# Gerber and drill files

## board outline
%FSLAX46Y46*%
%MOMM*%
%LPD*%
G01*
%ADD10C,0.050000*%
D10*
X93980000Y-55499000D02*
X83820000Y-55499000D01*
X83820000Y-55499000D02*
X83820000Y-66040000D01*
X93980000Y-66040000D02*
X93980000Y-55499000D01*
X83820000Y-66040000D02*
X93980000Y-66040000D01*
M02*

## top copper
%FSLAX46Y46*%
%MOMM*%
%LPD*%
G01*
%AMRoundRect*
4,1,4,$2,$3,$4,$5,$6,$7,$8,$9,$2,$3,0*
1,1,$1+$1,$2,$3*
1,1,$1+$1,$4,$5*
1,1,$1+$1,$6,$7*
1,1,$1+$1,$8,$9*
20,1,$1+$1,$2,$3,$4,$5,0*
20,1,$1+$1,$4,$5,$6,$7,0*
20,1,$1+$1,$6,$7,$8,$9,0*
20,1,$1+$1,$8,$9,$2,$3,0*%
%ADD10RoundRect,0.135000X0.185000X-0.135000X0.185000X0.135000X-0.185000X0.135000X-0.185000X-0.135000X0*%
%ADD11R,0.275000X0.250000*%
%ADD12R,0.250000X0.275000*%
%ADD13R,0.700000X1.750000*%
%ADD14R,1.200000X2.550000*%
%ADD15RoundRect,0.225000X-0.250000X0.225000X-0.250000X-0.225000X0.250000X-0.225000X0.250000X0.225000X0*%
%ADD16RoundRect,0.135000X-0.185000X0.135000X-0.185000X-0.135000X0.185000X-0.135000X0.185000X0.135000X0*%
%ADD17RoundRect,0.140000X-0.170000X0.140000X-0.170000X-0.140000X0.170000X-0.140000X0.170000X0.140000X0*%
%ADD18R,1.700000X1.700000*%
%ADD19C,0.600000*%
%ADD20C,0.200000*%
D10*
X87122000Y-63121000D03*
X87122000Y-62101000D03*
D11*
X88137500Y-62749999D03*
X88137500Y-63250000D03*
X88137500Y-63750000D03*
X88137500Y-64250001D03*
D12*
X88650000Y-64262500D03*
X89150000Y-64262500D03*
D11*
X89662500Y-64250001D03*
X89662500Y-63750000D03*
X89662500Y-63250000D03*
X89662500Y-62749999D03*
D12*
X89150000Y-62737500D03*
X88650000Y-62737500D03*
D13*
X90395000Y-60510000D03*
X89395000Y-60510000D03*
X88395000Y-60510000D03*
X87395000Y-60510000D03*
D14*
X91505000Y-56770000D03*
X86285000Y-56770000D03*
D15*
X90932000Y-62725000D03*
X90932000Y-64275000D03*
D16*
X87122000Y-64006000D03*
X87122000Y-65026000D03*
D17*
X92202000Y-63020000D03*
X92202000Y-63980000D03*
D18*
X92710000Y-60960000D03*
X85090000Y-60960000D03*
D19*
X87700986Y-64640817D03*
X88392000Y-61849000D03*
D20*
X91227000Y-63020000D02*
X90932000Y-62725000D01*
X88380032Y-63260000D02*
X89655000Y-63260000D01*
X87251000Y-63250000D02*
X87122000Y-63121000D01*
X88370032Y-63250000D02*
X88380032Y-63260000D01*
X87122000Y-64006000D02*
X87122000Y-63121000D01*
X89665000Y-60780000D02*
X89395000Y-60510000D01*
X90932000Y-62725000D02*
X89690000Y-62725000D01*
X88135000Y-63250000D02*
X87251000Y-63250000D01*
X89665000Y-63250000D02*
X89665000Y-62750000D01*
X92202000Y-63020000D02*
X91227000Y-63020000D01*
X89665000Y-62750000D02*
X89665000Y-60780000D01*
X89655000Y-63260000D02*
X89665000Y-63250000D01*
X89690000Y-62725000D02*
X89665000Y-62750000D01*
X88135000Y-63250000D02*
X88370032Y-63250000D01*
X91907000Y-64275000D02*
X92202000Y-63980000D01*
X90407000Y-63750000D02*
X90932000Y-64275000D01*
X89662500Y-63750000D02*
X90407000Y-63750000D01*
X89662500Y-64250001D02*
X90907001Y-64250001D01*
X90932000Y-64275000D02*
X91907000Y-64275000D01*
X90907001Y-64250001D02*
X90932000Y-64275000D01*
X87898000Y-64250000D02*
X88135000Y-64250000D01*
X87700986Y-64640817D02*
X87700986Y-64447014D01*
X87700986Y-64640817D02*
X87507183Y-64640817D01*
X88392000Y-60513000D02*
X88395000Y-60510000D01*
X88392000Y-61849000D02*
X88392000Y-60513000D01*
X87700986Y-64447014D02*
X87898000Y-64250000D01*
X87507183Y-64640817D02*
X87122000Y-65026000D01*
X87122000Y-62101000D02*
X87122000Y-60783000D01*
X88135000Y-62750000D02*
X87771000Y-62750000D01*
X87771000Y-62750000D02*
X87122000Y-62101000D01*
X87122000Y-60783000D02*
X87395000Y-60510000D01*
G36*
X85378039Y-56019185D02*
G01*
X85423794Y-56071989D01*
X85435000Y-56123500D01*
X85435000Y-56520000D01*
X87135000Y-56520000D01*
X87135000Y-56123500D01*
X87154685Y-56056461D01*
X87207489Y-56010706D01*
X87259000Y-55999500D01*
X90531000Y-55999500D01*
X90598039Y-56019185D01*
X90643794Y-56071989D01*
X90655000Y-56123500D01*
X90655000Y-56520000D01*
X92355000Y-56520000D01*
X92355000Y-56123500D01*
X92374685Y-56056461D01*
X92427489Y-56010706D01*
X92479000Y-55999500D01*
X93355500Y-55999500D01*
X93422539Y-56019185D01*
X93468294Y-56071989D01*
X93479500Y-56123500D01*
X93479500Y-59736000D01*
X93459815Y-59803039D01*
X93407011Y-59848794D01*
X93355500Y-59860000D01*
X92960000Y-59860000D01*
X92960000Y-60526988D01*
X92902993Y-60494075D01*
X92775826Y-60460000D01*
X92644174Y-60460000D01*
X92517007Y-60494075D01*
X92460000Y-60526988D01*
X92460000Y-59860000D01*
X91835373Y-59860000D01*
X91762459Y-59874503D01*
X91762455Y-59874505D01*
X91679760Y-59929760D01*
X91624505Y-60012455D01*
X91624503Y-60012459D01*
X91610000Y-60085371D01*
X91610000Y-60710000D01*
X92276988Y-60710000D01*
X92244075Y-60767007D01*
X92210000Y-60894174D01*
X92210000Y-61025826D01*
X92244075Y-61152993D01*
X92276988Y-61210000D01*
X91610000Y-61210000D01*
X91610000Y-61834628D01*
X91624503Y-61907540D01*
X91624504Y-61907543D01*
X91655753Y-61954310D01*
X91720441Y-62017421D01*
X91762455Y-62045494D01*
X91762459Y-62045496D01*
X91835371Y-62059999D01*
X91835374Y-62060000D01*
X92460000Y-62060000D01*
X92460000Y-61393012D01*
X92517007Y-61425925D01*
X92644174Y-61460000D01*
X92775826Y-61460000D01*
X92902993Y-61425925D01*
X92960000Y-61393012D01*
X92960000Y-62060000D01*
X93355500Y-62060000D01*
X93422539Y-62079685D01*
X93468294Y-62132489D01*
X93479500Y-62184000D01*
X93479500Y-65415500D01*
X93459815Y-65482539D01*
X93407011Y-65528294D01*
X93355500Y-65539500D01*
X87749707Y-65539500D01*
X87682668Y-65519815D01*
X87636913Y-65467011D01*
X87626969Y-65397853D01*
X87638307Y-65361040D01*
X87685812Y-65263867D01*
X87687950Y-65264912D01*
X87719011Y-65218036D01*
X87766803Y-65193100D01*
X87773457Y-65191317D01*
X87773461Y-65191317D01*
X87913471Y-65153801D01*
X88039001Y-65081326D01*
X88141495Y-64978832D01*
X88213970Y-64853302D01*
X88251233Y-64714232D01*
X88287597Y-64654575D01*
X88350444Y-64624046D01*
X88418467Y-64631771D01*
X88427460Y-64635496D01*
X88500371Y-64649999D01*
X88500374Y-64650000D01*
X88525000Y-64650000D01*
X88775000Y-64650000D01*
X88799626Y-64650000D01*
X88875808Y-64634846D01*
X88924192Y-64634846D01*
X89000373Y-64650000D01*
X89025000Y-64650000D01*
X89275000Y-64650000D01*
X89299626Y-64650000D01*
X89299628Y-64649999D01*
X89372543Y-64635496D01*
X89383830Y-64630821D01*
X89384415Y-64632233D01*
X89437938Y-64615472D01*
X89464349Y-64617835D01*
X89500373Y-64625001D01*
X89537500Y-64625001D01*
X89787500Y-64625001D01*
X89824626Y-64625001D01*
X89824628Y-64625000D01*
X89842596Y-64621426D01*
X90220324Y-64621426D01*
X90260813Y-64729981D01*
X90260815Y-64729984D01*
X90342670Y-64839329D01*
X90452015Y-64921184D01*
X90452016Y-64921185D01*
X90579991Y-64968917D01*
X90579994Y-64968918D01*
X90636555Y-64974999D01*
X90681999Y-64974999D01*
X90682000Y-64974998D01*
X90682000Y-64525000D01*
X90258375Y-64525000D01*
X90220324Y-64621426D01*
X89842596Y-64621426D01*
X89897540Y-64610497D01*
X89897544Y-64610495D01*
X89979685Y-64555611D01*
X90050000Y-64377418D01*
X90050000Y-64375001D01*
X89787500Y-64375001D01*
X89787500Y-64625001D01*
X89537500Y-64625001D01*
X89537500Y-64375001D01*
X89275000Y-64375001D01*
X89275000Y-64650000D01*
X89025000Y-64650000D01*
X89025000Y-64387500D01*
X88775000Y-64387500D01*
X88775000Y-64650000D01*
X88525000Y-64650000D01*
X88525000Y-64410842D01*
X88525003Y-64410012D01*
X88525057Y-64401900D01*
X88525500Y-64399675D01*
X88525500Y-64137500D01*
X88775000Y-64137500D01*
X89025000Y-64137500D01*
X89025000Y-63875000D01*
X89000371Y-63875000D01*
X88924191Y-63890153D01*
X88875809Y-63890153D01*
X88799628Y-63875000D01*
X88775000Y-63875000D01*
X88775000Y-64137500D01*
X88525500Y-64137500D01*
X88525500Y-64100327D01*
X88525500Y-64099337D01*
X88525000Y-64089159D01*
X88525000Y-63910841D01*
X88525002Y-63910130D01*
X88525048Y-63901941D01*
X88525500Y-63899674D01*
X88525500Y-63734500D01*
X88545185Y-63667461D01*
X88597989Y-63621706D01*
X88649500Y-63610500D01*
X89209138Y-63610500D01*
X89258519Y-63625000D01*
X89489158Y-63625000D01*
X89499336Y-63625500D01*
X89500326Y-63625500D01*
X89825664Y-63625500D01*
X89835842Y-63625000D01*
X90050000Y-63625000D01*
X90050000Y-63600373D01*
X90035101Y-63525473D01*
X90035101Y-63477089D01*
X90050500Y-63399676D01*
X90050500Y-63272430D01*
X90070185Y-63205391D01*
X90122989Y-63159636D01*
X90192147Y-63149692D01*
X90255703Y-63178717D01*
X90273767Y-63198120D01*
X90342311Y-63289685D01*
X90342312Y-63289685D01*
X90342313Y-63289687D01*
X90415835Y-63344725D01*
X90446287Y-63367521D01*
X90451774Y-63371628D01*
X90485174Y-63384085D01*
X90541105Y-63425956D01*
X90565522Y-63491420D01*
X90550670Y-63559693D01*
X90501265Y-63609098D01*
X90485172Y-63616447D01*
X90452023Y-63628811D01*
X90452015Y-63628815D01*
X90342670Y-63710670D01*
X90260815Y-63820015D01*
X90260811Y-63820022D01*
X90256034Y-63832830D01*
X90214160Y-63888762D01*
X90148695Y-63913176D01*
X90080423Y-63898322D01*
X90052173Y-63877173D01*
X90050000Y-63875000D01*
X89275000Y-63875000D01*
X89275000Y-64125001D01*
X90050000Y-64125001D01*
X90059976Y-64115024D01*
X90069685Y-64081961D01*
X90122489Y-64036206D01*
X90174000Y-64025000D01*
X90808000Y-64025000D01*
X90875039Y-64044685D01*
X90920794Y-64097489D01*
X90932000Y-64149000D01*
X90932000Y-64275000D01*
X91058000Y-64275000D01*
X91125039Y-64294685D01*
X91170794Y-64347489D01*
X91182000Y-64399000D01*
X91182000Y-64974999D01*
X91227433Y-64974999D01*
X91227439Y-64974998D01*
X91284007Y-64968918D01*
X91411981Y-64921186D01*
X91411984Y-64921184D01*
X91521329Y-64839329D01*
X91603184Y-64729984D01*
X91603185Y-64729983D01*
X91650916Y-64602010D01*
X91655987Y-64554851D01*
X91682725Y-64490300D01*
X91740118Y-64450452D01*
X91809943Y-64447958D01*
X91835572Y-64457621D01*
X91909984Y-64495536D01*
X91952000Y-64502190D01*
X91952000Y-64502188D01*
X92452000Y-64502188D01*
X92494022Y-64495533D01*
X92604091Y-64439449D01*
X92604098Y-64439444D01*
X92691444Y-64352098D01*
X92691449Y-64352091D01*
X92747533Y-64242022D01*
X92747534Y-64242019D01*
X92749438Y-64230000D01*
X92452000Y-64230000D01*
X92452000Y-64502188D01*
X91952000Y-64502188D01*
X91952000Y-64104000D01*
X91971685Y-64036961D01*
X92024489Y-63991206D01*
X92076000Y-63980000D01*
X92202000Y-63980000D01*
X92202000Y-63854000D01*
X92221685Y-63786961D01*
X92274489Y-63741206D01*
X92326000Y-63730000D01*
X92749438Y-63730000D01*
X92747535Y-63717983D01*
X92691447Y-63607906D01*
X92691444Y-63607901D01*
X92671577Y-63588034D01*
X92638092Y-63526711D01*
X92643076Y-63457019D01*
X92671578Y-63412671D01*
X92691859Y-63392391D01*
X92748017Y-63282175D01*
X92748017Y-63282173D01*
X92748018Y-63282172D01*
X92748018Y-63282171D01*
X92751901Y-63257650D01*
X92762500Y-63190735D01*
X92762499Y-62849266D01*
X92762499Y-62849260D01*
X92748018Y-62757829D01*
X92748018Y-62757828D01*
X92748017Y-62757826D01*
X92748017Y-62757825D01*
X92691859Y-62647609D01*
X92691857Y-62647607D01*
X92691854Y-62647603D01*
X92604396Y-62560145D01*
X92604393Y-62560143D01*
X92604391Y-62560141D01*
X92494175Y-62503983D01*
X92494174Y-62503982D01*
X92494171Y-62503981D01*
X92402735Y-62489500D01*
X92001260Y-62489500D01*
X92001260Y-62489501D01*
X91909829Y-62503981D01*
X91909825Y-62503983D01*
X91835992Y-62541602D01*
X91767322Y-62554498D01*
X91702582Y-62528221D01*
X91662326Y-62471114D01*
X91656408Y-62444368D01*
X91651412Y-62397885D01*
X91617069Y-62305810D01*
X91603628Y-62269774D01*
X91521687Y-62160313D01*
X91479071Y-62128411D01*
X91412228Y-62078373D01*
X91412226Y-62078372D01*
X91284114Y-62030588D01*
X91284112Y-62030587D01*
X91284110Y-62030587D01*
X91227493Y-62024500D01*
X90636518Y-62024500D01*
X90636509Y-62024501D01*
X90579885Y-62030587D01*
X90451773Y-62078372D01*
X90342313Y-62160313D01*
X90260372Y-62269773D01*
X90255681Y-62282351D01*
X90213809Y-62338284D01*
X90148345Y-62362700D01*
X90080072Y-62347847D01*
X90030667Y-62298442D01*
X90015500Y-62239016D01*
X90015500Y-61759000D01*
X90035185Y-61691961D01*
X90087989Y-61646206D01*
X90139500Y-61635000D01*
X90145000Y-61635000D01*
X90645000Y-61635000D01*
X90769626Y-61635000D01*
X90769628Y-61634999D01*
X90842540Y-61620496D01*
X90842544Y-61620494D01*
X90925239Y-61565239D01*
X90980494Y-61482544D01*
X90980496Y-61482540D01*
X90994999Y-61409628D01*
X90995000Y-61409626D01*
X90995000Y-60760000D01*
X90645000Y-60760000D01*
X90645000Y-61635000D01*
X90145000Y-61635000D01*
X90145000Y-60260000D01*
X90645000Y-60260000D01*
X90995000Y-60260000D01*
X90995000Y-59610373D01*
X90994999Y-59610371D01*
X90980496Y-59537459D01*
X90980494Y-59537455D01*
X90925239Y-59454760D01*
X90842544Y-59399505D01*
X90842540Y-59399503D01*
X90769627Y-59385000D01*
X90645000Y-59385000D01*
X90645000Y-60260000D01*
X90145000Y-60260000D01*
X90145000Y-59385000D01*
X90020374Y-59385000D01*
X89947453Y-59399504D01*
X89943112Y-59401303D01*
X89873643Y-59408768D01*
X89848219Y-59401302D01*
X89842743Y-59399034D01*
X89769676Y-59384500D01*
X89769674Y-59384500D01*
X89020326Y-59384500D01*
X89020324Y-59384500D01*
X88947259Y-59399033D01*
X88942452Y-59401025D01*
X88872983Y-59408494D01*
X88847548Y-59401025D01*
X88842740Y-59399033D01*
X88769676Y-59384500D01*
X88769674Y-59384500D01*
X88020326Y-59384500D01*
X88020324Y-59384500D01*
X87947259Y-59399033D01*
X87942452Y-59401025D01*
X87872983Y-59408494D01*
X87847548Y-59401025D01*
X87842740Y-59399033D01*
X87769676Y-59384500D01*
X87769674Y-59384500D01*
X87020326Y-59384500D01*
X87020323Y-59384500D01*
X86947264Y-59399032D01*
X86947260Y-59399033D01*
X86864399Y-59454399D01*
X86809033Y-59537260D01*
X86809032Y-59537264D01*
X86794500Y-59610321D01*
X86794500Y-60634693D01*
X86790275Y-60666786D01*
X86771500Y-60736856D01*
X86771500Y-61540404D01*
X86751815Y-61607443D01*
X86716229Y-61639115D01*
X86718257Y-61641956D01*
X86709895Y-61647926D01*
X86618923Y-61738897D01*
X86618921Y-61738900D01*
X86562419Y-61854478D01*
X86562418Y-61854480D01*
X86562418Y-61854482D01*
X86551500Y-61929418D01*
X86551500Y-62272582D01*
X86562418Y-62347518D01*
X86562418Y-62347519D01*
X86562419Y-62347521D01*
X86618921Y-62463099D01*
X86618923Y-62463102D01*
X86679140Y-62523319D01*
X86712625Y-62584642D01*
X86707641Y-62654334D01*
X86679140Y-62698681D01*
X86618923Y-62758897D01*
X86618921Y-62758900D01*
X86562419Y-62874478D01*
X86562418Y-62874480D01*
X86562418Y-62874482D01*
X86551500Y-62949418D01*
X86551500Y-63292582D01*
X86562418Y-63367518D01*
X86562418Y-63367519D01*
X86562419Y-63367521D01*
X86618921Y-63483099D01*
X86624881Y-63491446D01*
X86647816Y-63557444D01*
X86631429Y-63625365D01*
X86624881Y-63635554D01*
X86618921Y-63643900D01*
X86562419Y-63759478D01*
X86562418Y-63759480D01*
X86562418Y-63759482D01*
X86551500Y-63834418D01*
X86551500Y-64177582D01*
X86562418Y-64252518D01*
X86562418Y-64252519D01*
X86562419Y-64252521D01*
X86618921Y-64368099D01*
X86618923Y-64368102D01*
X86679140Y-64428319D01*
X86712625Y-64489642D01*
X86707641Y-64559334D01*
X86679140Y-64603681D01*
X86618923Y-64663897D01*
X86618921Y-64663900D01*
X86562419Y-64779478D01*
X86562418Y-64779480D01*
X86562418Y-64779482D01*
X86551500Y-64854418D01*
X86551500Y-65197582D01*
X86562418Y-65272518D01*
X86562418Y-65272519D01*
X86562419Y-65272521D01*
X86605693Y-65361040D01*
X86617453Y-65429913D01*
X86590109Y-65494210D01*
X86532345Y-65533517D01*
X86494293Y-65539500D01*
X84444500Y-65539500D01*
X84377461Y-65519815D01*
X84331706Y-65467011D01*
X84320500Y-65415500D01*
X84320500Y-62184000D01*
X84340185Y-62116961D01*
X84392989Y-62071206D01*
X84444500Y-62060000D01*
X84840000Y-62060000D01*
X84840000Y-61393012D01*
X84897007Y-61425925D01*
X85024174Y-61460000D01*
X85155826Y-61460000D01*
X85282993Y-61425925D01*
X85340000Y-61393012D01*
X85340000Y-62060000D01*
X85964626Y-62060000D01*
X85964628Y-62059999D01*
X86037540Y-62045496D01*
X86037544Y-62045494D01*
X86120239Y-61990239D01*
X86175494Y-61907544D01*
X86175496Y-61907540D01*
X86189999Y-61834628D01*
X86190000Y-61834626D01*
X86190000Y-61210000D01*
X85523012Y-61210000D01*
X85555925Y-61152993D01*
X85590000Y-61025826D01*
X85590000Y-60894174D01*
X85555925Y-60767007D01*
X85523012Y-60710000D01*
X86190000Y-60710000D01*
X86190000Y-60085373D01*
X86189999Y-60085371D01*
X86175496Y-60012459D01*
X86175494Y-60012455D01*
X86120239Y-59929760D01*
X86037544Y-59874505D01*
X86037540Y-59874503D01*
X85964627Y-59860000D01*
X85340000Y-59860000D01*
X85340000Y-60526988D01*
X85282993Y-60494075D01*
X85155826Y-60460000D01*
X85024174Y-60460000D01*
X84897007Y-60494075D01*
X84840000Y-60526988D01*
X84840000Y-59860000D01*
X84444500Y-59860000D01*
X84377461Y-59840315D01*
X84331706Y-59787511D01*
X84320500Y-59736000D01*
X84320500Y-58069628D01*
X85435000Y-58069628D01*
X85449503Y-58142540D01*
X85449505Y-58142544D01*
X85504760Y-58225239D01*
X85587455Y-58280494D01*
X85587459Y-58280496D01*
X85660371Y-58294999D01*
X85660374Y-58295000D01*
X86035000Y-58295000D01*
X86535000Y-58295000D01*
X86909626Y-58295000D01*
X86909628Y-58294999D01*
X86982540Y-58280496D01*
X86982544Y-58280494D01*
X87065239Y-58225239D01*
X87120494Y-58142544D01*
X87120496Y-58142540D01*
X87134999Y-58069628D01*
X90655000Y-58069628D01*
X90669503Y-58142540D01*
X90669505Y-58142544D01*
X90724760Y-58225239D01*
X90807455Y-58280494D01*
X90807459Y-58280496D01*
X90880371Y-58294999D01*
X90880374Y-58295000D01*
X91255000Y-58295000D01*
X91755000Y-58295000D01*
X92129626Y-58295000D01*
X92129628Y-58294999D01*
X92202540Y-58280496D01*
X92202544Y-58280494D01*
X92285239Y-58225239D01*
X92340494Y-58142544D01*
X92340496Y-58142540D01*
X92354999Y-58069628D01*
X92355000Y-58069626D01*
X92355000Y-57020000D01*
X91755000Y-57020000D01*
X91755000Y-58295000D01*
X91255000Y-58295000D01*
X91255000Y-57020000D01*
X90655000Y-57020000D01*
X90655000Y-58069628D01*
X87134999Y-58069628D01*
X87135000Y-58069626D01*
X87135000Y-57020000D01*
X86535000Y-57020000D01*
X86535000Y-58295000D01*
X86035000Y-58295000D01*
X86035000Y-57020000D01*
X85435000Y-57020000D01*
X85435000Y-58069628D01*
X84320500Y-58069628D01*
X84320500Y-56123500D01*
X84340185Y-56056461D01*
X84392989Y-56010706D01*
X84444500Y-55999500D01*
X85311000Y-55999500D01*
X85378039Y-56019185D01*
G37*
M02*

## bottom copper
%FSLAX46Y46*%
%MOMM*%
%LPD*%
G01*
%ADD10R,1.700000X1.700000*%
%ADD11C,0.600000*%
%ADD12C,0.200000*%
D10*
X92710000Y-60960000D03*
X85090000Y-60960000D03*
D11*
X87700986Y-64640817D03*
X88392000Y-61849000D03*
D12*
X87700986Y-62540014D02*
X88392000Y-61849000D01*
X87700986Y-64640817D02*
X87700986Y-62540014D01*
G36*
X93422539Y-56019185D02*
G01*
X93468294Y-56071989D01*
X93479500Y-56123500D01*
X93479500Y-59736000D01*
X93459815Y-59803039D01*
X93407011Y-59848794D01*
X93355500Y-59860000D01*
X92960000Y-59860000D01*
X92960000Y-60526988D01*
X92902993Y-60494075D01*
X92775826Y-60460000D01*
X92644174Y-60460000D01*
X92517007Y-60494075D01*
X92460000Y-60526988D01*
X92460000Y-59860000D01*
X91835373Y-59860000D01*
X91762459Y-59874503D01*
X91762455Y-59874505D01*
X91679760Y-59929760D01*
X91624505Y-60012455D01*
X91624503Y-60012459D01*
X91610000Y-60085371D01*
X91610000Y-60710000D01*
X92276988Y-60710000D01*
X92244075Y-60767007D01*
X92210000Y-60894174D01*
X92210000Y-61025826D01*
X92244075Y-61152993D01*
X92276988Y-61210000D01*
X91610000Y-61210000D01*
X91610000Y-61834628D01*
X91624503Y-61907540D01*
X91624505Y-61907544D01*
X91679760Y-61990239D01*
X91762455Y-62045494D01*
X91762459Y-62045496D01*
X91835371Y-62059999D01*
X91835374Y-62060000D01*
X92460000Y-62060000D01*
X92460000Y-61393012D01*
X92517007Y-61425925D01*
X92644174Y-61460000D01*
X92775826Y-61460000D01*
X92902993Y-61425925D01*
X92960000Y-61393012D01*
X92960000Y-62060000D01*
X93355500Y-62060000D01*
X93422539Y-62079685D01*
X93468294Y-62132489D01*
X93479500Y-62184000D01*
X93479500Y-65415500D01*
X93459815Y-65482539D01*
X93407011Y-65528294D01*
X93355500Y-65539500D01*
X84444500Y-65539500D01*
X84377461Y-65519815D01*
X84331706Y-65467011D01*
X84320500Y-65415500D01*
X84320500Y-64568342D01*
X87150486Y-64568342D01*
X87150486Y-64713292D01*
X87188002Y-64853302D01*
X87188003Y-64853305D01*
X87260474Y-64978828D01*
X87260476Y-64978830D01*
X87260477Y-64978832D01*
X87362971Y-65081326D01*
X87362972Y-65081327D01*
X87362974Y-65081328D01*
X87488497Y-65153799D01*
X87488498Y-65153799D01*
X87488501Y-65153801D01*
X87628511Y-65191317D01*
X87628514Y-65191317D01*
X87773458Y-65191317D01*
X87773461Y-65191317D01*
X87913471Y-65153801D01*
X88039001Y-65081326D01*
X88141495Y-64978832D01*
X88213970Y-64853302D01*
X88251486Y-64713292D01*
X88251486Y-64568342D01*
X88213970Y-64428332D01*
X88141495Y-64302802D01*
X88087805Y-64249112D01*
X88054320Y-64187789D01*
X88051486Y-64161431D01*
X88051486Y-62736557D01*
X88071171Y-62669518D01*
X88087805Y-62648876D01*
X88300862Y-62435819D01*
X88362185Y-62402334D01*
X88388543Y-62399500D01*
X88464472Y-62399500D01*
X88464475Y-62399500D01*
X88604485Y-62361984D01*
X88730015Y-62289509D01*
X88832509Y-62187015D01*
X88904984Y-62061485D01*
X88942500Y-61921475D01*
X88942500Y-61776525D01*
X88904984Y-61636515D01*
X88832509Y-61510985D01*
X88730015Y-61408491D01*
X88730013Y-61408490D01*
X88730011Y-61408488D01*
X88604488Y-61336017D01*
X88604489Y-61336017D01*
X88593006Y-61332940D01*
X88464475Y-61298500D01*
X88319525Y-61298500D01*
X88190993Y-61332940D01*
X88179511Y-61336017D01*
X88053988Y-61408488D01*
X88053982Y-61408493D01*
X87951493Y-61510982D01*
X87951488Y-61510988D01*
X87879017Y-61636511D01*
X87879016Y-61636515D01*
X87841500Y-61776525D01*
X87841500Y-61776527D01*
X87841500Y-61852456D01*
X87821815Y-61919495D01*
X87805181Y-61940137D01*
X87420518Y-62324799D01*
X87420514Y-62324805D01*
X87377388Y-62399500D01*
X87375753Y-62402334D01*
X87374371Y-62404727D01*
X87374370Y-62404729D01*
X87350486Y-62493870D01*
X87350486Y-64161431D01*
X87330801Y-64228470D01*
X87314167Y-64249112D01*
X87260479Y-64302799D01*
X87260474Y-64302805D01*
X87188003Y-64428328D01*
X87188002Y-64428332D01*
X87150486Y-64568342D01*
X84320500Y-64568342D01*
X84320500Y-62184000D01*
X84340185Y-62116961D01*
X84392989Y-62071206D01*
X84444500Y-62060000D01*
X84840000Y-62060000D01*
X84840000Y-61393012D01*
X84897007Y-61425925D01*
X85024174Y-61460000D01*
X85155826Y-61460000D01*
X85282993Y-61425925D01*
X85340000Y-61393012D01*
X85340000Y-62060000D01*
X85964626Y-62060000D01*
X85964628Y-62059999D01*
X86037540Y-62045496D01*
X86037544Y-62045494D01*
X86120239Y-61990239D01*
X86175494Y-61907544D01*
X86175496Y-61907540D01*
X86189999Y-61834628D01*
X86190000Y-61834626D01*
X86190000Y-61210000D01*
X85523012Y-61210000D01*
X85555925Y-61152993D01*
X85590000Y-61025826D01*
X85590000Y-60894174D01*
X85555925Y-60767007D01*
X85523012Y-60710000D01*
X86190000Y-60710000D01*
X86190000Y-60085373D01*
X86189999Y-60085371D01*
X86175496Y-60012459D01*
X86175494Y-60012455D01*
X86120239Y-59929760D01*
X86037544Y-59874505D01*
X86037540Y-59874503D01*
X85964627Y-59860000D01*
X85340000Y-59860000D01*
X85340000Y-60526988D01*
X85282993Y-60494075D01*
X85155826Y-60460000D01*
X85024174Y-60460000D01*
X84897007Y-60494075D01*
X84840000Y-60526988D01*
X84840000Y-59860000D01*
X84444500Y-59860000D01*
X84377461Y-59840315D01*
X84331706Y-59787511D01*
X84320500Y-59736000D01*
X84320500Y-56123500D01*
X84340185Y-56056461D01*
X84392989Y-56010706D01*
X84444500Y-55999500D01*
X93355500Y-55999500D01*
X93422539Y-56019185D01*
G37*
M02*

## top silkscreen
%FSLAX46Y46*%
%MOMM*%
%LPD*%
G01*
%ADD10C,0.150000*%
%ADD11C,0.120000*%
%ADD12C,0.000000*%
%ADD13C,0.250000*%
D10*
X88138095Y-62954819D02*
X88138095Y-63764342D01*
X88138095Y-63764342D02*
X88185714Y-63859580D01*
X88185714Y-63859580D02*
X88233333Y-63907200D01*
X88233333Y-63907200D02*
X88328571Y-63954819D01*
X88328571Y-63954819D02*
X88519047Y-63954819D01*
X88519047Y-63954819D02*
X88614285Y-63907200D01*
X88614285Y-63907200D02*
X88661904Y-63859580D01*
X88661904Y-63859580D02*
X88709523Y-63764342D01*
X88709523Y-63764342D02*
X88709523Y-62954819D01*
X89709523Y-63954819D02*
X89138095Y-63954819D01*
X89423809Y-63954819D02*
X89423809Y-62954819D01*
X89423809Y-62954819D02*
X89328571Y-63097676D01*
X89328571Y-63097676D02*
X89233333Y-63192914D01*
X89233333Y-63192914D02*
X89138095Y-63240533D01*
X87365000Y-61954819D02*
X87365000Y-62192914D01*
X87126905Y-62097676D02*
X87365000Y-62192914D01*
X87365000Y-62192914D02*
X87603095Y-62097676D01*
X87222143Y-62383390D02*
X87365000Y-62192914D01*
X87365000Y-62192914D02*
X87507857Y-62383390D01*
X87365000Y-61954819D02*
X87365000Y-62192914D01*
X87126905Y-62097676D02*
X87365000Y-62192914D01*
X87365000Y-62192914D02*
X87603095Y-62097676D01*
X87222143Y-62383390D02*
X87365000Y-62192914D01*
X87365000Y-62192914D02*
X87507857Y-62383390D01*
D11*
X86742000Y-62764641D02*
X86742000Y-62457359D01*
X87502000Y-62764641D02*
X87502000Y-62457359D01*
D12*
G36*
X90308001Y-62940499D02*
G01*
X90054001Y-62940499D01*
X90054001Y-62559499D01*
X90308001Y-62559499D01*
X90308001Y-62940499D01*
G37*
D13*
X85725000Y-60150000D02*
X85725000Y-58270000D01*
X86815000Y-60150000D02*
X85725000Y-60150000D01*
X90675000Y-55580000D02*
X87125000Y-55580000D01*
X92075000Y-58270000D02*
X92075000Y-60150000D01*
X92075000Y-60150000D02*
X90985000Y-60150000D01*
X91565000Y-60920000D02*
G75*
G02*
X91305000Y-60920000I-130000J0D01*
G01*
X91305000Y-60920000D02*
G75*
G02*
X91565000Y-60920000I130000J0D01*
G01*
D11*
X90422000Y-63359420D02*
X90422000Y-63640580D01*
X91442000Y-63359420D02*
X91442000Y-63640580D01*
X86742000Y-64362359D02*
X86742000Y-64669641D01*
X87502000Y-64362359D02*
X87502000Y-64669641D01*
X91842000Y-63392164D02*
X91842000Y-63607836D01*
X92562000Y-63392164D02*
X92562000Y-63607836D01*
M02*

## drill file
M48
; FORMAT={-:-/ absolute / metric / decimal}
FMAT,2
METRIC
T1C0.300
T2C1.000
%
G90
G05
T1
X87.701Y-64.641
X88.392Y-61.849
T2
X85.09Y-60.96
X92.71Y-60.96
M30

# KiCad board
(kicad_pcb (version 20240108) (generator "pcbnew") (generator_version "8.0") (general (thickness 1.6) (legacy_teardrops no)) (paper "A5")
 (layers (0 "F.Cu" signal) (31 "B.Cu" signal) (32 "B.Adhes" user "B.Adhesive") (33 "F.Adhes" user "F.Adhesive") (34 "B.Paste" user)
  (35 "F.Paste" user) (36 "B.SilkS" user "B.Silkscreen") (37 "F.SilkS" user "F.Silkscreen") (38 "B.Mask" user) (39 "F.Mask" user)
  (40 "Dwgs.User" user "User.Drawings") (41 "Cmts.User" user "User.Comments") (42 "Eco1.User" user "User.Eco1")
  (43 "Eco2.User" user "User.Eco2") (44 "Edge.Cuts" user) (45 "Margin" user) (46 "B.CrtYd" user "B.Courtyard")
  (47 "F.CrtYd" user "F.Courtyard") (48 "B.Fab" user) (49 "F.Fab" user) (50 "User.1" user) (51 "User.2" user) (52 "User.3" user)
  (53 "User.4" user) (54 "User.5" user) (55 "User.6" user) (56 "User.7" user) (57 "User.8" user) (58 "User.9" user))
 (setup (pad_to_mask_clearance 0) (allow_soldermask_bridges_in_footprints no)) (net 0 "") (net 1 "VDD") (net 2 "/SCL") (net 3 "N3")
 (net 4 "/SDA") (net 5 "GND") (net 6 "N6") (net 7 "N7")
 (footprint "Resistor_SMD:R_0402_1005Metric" (layer "F.Cu") (at 87.122 62.611 90)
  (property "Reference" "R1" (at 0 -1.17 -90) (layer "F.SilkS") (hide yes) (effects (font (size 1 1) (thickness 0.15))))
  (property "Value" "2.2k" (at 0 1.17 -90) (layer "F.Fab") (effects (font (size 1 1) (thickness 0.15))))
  (fp_line (start -0.153641 -0.38) (end 0.153641 -0.38) (stroke (width 0.12) (type solid)) (layer "F.SilkS"))
  (fp_line (start -0.153641 0.38) (end 0.153641 0.38) (stroke (width 0.12) (type solid)) (layer "F.SilkS"))
  (pad "1" smd roundrect (at -0.51 0 90) (size 0.54 0.64) (layers "F.Cu" "F.Paste" "F.Mask") (roundrect_rratio 0.25) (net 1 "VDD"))
  (pad "2" smd roundrect (at 0.51 0 90) (size 0.54 0.64) (layers "F.Cu" "F.Paste" "F.Mask") (roundrect_rratio 0.25) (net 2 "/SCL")))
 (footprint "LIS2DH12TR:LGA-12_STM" (layer "F.Cu") (at 88.9 63.5)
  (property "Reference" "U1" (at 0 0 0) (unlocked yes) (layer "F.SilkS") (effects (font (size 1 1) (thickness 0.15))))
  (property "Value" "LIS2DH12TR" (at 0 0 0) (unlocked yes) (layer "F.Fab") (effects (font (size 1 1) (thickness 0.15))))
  (fp_poly
   (pts (xy 1.408001 -0.940501) (xy 1.408001 -0.559501) (xy 1.154001 -0.559501) (xy 1.154001 -0.940501)) (stroke (width 0) (type solid))
   (fill solid) (layer "F.SilkS"))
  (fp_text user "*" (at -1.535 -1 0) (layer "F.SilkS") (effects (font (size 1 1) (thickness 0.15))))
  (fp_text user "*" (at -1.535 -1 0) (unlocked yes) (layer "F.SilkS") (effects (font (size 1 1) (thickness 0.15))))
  (pad "1" smd rect (at -0.7625 -0.750001 90) (size 0.25 0.275) (layers "F.Cu" "F.Paste" "F.Mask") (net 2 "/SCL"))
  (pad "2" smd rect (at -0.7625 -0.25 90) (size 0.25 0.275) (layers "F.Cu" "F.Paste" "F.Mask") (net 1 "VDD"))
  (pad "3" smd rect (at -0.7625 0.25 90) (size 0.25 0.275) (layers "F.Cu" "F.Paste" "F.Mask") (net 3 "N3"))
  (pad "4" smd rect (at -0.7625 0.750001 90) (size 0.25 0.275) (layers "F.Cu" "F.Paste" "F.Mask") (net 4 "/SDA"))
  (pad "5" smd rect (at -0.25 0.7625) (size 0.25 0.275) (layers "F.Cu" "F.Paste" "F.Mask") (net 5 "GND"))
  (pad "6" smd rect (at 0.25 0.7625) (size 0.25 0.275) (layers "F.Cu" "F.Paste" "F.Mask") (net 5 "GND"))
  (pad "7" smd rect (at 0.7625 0.750001 90) (size 0.25 0.275) (layers "F.Cu" "F.Paste" "F.Mask") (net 5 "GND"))
  (pad "8" smd rect (at 0.7625 0.25 90) (size 0.25 0.275) (layers "F.Cu" "F.Paste" "F.Mask") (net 5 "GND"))
  (pad "9" smd rect (at 0.7625 -0.25 90) (size 0.25 0.275) (layers "F.Cu" "F.Paste" "F.Mask") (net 1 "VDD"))
  (pad "10" smd rect (at 0.7625 -0.750001 90) (size 0.25 0.275) (layers "F.Cu" "F.Paste" "F.Mask") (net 1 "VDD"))
  (pad "11" smd rect (at 0.25 -0.7625) (size 0.25 0.275) (layers "F.Cu" "F.Paste" "F.Mask") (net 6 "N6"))
  (pad "12" smd rect (at -0.25 -0.7625) (size 0.25 0.275) (layers "F.Cu" "F.Paste" "F.Mask") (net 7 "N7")))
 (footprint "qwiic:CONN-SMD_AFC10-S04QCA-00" (layer "F.Cu") (at 88.895 58.64 180)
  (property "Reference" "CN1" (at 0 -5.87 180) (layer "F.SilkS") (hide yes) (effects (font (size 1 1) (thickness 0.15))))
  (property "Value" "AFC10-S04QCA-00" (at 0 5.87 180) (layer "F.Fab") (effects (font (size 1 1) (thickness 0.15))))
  (fp_line (start 3.17 -1.51) (end 3.17 0.37) (stroke (width 0.25) (type solid)) (layer "F.SilkS"))
  (fp_line (start 2.08 -1.51) (end 3.17 -1.51) (stroke (width 0.25) (type solid)) (layer "F.SilkS"))
  (fp_line (start -1.78 3.06) (end 1.77 3.06) (stroke (width 0.25) (type solid)) (layer "F.SilkS"))
  (fp_line (start -3.18 0.37) (end -3.18 -1.51) (stroke (width 0.25) (type solid)) (layer "F.SilkS"))
  (fp_line (start -3.18 -1.51) (end -2.09 -1.51) (stroke (width 0.25) (type solid)) (layer "F.SilkS"))
  (fp_circle (center -2.54 -2.28) (end -2.41 -2.28) (stroke (width 0.25) (type solid)) (fill none) (layer "F.SilkS"))
  (pad "1" smd rect (at -1.5 -1.87 180) (size 0.7 1.75) (layers "F.Cu" "F.Paste" "F.Mask") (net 5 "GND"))
  (pad "2" smd rect (at -0.5 -1.87 180) (size 0.7 1.75) (layers "F.Cu" "F.Paste" "F.Mask") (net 1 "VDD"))
  (pad "3" smd rect (at 0.5 -1.87 180) (size 0.7 1.75) (layers "F.Cu" "F.Paste" "F.Mask") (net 4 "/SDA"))
  (pad "4" smd rect (at 1.5 -1.87 180) (size 0.7 1.75) (layers "F.Cu" "F.Paste" "F.Mask") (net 2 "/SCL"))
  (pad "5" smd rect (at -2.61 1.87 180) (size 1.2 2.55) (layers "F.Cu" "F.Paste" "F.Mask") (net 5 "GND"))
  (pad "6" smd rect (at 2.61 1.87 180) (size 1.2 2.55) (layers "F.Cu" "F.Paste" "F.Mask") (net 5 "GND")))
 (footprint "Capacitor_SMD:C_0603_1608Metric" (layer "F.Cu") (at 90.932 63.5 -90)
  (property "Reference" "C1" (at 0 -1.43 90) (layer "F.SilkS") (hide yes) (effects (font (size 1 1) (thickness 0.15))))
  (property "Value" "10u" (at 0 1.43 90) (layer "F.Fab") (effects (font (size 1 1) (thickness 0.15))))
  (fp_line (start -0.14058 0.51) (end 0.14058 0.51) (stroke (width 0.12) (type solid)) (layer "F.SilkS"))
  (fp_line (start -0.14058 -0.51) (end 0.14058 -0.51) (stroke (width 0.12) (type solid)) (layer "F.SilkS"))
  (pad "1" smd roundrect (at -0.775 0 270) (size 0.9 0.95) (layers "F.Cu" "F.Paste" "F.Mask") (roundrect_rratio 0.25) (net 1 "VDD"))
  (pad "2" smd roundrect (at 0.775 0 270) (size 0.9 0.95) (layers "F.Cu" "F.Paste" "F.Mask") (roundrect_rratio 0.25) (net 5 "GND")))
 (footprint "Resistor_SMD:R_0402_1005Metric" (layer "F.Cu") (at 87.122 64.516 -90)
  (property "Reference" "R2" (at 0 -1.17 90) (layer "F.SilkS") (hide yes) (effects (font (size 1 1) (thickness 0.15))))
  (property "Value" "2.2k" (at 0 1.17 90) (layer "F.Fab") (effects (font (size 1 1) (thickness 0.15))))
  (fp_line (start -0.153641 0.38) (end 0.153641 0.38) (stroke (width 0.12) (type solid)) (layer "F.SilkS"))
  (fp_line (start -0.153641 -0.38) (end 0.153641 -0.38) (stroke (width 0.12) (type solid)) (layer "F.SilkS"))
  (pad "1" smd roundrect (at -0.51 0 270) (size 0.54 0.64) (layers "F.Cu" "F.Paste" "F.Mask") (roundrect_rratio 0.25) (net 1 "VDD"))
  (pad "2" smd roundrect (at 0.51 0 270) (size 0.54 0.64) (layers "F.Cu" "F.Paste" "F.Mask") (roundrect_rratio 0.25) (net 4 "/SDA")))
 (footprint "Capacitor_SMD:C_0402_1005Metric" (layer "F.Cu") (at 92.202 63.5 -90)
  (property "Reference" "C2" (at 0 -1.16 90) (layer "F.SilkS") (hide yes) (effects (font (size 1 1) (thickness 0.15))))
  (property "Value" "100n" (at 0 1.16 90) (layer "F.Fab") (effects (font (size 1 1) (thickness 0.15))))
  (fp_line (start -0.107836 0.36) (end 0.107836 0.36) (stroke (width 0.12) (type solid)) (layer "F.SilkS"))
  (fp_line (start -0.107836 -0.36) (end 0.107836 -0.36) (stroke (width 0.12) (type solid)) (layer "F.SilkS"))
  (pad "1" smd roundrect (at -0.48 0 270) (size 0.56 0.62) (layers "F.Cu" "F.Paste" "F.Mask") (roundrect_rratio 0.25) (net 1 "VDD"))
  (pad "2" smd roundrect (at 0.48 0 270) (size 0.56 0.62) (layers "F.Cu" "F.Paste" "F.Mask") (roundrect_rratio 0.25) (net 5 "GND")))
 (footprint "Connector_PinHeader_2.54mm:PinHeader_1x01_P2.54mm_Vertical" (layer "B.Cu") (at 92.71 60.96 180)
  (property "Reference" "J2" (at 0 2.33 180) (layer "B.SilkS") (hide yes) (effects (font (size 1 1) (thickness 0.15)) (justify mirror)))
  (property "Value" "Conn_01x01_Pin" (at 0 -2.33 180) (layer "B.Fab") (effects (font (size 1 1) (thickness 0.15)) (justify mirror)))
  (pad "1" thru_hole rect (at 0 0 180) (size 1.7 1.7) (drill 1) (layers "*.Cu" "*.Mask") (remove_unused_layers no) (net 5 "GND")))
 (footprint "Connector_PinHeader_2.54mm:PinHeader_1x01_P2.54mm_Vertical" (layer "B.Cu") (at 85.09 60.96 180)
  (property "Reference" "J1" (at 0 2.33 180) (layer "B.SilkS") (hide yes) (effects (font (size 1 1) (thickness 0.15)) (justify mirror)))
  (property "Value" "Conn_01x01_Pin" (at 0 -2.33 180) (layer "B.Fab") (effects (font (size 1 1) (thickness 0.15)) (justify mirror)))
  (pad "1" thru_hole rect (at 0 0 180) (size 1.7 1.7) (drill 1) (layers "*.Cu" "*.Mask") (remove_unused_layers no) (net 5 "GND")))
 (gr_line (start 93.98 55.499) (end 83.82 55.499) (stroke (width 0.05) (type default)) (layer "Edge.Cuts"))
 (gr_line (start 83.82 55.499) (end 83.82 66.04) (stroke (width 0.05) (type default)) (layer "Edge.Cuts"))
 (gr_line (start 93.98 66.04) (end 93.98 55.499) (stroke (width 0.05) (type default)) (layer "Edge.Cuts"))
 (gr_line (start 83.82 66.04) (end 93.98 66.04) (stroke (width 0.05) (type default)) (layer "Edge.Cuts"))
 (segment (start 91.227 63.02) (end 90.932 62.725) (width 0.2) (layer "F.Cu") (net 1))
 (segment (start 88.380032 63.26) (end 89.655 63.26) (width 0.2) (layer "F.Cu") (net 1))
 (segment (start 87.251 63.25) (end 87.122 63.121) (width 0.2) (layer "F.Cu") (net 1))
 (segment (start 88.370032 63.25) (end 88.380032 63.26) (width 0.2) (layer "F.Cu") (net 1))
 (segment (start 87.122 64.006) (end 87.122 63.121) (width 0.2) (layer "F.Cu") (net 1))
 (segment (start 89.665 60.78) (end 89.395 60.51) (width 0.2) (layer "F.Cu") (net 1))
 (segment (start 90.932 62.725) (end 89.69 62.725) (width 0.2) (layer "F.Cu") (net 1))
 (segment (start 88.135 63.25) (end 87.251 63.25) (width 0.2) (layer "F.Cu") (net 1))
 (segment (start 89.665 63.25) (end 89.665 62.75) (width 0.2) (layer "F.Cu") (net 1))
 (segment (start 92.202 63.02) (end 91.227 63.02) (width 0.2) (layer "F.Cu") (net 1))
 (segment (start 89.665 62.75) (end 89.665 60.78) (width 0.2) (layer "F.Cu") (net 1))
 (segment (start 89.655 63.26) (end 89.665 63.25) (width 0.2) (layer "F.Cu") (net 1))
 (segment (start 89.69 62.725) (end 89.665 62.75) (width 0.2) (layer "F.Cu") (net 1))
 (segment (start 88.135 63.25) (end 88.370032 63.25) (width 0.2) (layer "F.Cu") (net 1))
 (segment (start 91.907 64.275) (end 92.202 63.98) (width 0.2) (layer "F.Cu") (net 5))
 (segment (start 90.407 63.75) (end 90.932 64.275) (width 0.2) (layer "F.Cu") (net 5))
 (segment (start 89.6625 63.75) (end 90.407 63.75) (width 0.2) (layer "F.Cu") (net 5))
 (segment (start 89.6625 64.250001) (end 90.907001 64.250001) (width 0.2) (layer "F.Cu") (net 5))
 (segment (start 90.932 64.275) (end 91.907 64.275) (width 0.2) (layer "F.Cu") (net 5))
 (segment (start 90.907001 64.250001) (end 90.932 64.275) (width 0.2) (layer "F.Cu") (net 5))
 (segment (start 87.898 64.25) (end 88.135 64.25) (width 0.2) (layer "F.Cu") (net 4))
 (segment (start 87.700986 64.640817) (end 87.700986 64.447014) (width 0.2) (layer "F.Cu") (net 4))
 (segment (start 87.700986 64.640817) (end 87.507183 64.640817) (width 0.2) (layer "F.Cu") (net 4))
 (segment (start 88.392 60.513) (end 88.395 60.51) (width 0.2) (layer "F.Cu") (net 4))
 (segment (start 88.392 61.849) (end 88.392 60.513) (width 0.2) (layer "F.Cu") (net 4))
 (segment (start 87.700986 64.447014) (end 87.898 64.25) (width 0.2) (layer "F.Cu") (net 4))
 (segment (start 87.507183 64.640817) (end 87.122 65.026) (width 0.2) (layer "F.Cu") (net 4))
 (via (at 87.700986 64.640817) (size 0.6) (drill 0.3) (layers "F.Cu" "B.Cu") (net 4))
 (via (at 88.392 61.849) (size 0.6) (drill 0.3) (layers "F.Cu" "B.Cu") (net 4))
 (segment (start 87.700986 62.540014) (end 88.392 61.849) (width 0.2) (layer "B.Cu") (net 4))
 (segment (start 87.700986 64.640817) (end 87.700986 62.540014) (width 0.2) (layer "B.Cu") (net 4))
 (segment (start 87.122 62.101) (end 87.122 60.783) (width 0.2) (layer "F.Cu") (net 2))
 (segment (start 88.135 62.75) (end 87.771 62.75) (width 0.2) (layer "F.Cu") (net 2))
 (segment (start 87.771 62.75) (end 87.122 62.101) (width 0.2) (layer "F.Cu") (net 2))
 (segment (start 87.122 60.783) (end 87.395 60.51) (width 0.2) (layer "F.Cu") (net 2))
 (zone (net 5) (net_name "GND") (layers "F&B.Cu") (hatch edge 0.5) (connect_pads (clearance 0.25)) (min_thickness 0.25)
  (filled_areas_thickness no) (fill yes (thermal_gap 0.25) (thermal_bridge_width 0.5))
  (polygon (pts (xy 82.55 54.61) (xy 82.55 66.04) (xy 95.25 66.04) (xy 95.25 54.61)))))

